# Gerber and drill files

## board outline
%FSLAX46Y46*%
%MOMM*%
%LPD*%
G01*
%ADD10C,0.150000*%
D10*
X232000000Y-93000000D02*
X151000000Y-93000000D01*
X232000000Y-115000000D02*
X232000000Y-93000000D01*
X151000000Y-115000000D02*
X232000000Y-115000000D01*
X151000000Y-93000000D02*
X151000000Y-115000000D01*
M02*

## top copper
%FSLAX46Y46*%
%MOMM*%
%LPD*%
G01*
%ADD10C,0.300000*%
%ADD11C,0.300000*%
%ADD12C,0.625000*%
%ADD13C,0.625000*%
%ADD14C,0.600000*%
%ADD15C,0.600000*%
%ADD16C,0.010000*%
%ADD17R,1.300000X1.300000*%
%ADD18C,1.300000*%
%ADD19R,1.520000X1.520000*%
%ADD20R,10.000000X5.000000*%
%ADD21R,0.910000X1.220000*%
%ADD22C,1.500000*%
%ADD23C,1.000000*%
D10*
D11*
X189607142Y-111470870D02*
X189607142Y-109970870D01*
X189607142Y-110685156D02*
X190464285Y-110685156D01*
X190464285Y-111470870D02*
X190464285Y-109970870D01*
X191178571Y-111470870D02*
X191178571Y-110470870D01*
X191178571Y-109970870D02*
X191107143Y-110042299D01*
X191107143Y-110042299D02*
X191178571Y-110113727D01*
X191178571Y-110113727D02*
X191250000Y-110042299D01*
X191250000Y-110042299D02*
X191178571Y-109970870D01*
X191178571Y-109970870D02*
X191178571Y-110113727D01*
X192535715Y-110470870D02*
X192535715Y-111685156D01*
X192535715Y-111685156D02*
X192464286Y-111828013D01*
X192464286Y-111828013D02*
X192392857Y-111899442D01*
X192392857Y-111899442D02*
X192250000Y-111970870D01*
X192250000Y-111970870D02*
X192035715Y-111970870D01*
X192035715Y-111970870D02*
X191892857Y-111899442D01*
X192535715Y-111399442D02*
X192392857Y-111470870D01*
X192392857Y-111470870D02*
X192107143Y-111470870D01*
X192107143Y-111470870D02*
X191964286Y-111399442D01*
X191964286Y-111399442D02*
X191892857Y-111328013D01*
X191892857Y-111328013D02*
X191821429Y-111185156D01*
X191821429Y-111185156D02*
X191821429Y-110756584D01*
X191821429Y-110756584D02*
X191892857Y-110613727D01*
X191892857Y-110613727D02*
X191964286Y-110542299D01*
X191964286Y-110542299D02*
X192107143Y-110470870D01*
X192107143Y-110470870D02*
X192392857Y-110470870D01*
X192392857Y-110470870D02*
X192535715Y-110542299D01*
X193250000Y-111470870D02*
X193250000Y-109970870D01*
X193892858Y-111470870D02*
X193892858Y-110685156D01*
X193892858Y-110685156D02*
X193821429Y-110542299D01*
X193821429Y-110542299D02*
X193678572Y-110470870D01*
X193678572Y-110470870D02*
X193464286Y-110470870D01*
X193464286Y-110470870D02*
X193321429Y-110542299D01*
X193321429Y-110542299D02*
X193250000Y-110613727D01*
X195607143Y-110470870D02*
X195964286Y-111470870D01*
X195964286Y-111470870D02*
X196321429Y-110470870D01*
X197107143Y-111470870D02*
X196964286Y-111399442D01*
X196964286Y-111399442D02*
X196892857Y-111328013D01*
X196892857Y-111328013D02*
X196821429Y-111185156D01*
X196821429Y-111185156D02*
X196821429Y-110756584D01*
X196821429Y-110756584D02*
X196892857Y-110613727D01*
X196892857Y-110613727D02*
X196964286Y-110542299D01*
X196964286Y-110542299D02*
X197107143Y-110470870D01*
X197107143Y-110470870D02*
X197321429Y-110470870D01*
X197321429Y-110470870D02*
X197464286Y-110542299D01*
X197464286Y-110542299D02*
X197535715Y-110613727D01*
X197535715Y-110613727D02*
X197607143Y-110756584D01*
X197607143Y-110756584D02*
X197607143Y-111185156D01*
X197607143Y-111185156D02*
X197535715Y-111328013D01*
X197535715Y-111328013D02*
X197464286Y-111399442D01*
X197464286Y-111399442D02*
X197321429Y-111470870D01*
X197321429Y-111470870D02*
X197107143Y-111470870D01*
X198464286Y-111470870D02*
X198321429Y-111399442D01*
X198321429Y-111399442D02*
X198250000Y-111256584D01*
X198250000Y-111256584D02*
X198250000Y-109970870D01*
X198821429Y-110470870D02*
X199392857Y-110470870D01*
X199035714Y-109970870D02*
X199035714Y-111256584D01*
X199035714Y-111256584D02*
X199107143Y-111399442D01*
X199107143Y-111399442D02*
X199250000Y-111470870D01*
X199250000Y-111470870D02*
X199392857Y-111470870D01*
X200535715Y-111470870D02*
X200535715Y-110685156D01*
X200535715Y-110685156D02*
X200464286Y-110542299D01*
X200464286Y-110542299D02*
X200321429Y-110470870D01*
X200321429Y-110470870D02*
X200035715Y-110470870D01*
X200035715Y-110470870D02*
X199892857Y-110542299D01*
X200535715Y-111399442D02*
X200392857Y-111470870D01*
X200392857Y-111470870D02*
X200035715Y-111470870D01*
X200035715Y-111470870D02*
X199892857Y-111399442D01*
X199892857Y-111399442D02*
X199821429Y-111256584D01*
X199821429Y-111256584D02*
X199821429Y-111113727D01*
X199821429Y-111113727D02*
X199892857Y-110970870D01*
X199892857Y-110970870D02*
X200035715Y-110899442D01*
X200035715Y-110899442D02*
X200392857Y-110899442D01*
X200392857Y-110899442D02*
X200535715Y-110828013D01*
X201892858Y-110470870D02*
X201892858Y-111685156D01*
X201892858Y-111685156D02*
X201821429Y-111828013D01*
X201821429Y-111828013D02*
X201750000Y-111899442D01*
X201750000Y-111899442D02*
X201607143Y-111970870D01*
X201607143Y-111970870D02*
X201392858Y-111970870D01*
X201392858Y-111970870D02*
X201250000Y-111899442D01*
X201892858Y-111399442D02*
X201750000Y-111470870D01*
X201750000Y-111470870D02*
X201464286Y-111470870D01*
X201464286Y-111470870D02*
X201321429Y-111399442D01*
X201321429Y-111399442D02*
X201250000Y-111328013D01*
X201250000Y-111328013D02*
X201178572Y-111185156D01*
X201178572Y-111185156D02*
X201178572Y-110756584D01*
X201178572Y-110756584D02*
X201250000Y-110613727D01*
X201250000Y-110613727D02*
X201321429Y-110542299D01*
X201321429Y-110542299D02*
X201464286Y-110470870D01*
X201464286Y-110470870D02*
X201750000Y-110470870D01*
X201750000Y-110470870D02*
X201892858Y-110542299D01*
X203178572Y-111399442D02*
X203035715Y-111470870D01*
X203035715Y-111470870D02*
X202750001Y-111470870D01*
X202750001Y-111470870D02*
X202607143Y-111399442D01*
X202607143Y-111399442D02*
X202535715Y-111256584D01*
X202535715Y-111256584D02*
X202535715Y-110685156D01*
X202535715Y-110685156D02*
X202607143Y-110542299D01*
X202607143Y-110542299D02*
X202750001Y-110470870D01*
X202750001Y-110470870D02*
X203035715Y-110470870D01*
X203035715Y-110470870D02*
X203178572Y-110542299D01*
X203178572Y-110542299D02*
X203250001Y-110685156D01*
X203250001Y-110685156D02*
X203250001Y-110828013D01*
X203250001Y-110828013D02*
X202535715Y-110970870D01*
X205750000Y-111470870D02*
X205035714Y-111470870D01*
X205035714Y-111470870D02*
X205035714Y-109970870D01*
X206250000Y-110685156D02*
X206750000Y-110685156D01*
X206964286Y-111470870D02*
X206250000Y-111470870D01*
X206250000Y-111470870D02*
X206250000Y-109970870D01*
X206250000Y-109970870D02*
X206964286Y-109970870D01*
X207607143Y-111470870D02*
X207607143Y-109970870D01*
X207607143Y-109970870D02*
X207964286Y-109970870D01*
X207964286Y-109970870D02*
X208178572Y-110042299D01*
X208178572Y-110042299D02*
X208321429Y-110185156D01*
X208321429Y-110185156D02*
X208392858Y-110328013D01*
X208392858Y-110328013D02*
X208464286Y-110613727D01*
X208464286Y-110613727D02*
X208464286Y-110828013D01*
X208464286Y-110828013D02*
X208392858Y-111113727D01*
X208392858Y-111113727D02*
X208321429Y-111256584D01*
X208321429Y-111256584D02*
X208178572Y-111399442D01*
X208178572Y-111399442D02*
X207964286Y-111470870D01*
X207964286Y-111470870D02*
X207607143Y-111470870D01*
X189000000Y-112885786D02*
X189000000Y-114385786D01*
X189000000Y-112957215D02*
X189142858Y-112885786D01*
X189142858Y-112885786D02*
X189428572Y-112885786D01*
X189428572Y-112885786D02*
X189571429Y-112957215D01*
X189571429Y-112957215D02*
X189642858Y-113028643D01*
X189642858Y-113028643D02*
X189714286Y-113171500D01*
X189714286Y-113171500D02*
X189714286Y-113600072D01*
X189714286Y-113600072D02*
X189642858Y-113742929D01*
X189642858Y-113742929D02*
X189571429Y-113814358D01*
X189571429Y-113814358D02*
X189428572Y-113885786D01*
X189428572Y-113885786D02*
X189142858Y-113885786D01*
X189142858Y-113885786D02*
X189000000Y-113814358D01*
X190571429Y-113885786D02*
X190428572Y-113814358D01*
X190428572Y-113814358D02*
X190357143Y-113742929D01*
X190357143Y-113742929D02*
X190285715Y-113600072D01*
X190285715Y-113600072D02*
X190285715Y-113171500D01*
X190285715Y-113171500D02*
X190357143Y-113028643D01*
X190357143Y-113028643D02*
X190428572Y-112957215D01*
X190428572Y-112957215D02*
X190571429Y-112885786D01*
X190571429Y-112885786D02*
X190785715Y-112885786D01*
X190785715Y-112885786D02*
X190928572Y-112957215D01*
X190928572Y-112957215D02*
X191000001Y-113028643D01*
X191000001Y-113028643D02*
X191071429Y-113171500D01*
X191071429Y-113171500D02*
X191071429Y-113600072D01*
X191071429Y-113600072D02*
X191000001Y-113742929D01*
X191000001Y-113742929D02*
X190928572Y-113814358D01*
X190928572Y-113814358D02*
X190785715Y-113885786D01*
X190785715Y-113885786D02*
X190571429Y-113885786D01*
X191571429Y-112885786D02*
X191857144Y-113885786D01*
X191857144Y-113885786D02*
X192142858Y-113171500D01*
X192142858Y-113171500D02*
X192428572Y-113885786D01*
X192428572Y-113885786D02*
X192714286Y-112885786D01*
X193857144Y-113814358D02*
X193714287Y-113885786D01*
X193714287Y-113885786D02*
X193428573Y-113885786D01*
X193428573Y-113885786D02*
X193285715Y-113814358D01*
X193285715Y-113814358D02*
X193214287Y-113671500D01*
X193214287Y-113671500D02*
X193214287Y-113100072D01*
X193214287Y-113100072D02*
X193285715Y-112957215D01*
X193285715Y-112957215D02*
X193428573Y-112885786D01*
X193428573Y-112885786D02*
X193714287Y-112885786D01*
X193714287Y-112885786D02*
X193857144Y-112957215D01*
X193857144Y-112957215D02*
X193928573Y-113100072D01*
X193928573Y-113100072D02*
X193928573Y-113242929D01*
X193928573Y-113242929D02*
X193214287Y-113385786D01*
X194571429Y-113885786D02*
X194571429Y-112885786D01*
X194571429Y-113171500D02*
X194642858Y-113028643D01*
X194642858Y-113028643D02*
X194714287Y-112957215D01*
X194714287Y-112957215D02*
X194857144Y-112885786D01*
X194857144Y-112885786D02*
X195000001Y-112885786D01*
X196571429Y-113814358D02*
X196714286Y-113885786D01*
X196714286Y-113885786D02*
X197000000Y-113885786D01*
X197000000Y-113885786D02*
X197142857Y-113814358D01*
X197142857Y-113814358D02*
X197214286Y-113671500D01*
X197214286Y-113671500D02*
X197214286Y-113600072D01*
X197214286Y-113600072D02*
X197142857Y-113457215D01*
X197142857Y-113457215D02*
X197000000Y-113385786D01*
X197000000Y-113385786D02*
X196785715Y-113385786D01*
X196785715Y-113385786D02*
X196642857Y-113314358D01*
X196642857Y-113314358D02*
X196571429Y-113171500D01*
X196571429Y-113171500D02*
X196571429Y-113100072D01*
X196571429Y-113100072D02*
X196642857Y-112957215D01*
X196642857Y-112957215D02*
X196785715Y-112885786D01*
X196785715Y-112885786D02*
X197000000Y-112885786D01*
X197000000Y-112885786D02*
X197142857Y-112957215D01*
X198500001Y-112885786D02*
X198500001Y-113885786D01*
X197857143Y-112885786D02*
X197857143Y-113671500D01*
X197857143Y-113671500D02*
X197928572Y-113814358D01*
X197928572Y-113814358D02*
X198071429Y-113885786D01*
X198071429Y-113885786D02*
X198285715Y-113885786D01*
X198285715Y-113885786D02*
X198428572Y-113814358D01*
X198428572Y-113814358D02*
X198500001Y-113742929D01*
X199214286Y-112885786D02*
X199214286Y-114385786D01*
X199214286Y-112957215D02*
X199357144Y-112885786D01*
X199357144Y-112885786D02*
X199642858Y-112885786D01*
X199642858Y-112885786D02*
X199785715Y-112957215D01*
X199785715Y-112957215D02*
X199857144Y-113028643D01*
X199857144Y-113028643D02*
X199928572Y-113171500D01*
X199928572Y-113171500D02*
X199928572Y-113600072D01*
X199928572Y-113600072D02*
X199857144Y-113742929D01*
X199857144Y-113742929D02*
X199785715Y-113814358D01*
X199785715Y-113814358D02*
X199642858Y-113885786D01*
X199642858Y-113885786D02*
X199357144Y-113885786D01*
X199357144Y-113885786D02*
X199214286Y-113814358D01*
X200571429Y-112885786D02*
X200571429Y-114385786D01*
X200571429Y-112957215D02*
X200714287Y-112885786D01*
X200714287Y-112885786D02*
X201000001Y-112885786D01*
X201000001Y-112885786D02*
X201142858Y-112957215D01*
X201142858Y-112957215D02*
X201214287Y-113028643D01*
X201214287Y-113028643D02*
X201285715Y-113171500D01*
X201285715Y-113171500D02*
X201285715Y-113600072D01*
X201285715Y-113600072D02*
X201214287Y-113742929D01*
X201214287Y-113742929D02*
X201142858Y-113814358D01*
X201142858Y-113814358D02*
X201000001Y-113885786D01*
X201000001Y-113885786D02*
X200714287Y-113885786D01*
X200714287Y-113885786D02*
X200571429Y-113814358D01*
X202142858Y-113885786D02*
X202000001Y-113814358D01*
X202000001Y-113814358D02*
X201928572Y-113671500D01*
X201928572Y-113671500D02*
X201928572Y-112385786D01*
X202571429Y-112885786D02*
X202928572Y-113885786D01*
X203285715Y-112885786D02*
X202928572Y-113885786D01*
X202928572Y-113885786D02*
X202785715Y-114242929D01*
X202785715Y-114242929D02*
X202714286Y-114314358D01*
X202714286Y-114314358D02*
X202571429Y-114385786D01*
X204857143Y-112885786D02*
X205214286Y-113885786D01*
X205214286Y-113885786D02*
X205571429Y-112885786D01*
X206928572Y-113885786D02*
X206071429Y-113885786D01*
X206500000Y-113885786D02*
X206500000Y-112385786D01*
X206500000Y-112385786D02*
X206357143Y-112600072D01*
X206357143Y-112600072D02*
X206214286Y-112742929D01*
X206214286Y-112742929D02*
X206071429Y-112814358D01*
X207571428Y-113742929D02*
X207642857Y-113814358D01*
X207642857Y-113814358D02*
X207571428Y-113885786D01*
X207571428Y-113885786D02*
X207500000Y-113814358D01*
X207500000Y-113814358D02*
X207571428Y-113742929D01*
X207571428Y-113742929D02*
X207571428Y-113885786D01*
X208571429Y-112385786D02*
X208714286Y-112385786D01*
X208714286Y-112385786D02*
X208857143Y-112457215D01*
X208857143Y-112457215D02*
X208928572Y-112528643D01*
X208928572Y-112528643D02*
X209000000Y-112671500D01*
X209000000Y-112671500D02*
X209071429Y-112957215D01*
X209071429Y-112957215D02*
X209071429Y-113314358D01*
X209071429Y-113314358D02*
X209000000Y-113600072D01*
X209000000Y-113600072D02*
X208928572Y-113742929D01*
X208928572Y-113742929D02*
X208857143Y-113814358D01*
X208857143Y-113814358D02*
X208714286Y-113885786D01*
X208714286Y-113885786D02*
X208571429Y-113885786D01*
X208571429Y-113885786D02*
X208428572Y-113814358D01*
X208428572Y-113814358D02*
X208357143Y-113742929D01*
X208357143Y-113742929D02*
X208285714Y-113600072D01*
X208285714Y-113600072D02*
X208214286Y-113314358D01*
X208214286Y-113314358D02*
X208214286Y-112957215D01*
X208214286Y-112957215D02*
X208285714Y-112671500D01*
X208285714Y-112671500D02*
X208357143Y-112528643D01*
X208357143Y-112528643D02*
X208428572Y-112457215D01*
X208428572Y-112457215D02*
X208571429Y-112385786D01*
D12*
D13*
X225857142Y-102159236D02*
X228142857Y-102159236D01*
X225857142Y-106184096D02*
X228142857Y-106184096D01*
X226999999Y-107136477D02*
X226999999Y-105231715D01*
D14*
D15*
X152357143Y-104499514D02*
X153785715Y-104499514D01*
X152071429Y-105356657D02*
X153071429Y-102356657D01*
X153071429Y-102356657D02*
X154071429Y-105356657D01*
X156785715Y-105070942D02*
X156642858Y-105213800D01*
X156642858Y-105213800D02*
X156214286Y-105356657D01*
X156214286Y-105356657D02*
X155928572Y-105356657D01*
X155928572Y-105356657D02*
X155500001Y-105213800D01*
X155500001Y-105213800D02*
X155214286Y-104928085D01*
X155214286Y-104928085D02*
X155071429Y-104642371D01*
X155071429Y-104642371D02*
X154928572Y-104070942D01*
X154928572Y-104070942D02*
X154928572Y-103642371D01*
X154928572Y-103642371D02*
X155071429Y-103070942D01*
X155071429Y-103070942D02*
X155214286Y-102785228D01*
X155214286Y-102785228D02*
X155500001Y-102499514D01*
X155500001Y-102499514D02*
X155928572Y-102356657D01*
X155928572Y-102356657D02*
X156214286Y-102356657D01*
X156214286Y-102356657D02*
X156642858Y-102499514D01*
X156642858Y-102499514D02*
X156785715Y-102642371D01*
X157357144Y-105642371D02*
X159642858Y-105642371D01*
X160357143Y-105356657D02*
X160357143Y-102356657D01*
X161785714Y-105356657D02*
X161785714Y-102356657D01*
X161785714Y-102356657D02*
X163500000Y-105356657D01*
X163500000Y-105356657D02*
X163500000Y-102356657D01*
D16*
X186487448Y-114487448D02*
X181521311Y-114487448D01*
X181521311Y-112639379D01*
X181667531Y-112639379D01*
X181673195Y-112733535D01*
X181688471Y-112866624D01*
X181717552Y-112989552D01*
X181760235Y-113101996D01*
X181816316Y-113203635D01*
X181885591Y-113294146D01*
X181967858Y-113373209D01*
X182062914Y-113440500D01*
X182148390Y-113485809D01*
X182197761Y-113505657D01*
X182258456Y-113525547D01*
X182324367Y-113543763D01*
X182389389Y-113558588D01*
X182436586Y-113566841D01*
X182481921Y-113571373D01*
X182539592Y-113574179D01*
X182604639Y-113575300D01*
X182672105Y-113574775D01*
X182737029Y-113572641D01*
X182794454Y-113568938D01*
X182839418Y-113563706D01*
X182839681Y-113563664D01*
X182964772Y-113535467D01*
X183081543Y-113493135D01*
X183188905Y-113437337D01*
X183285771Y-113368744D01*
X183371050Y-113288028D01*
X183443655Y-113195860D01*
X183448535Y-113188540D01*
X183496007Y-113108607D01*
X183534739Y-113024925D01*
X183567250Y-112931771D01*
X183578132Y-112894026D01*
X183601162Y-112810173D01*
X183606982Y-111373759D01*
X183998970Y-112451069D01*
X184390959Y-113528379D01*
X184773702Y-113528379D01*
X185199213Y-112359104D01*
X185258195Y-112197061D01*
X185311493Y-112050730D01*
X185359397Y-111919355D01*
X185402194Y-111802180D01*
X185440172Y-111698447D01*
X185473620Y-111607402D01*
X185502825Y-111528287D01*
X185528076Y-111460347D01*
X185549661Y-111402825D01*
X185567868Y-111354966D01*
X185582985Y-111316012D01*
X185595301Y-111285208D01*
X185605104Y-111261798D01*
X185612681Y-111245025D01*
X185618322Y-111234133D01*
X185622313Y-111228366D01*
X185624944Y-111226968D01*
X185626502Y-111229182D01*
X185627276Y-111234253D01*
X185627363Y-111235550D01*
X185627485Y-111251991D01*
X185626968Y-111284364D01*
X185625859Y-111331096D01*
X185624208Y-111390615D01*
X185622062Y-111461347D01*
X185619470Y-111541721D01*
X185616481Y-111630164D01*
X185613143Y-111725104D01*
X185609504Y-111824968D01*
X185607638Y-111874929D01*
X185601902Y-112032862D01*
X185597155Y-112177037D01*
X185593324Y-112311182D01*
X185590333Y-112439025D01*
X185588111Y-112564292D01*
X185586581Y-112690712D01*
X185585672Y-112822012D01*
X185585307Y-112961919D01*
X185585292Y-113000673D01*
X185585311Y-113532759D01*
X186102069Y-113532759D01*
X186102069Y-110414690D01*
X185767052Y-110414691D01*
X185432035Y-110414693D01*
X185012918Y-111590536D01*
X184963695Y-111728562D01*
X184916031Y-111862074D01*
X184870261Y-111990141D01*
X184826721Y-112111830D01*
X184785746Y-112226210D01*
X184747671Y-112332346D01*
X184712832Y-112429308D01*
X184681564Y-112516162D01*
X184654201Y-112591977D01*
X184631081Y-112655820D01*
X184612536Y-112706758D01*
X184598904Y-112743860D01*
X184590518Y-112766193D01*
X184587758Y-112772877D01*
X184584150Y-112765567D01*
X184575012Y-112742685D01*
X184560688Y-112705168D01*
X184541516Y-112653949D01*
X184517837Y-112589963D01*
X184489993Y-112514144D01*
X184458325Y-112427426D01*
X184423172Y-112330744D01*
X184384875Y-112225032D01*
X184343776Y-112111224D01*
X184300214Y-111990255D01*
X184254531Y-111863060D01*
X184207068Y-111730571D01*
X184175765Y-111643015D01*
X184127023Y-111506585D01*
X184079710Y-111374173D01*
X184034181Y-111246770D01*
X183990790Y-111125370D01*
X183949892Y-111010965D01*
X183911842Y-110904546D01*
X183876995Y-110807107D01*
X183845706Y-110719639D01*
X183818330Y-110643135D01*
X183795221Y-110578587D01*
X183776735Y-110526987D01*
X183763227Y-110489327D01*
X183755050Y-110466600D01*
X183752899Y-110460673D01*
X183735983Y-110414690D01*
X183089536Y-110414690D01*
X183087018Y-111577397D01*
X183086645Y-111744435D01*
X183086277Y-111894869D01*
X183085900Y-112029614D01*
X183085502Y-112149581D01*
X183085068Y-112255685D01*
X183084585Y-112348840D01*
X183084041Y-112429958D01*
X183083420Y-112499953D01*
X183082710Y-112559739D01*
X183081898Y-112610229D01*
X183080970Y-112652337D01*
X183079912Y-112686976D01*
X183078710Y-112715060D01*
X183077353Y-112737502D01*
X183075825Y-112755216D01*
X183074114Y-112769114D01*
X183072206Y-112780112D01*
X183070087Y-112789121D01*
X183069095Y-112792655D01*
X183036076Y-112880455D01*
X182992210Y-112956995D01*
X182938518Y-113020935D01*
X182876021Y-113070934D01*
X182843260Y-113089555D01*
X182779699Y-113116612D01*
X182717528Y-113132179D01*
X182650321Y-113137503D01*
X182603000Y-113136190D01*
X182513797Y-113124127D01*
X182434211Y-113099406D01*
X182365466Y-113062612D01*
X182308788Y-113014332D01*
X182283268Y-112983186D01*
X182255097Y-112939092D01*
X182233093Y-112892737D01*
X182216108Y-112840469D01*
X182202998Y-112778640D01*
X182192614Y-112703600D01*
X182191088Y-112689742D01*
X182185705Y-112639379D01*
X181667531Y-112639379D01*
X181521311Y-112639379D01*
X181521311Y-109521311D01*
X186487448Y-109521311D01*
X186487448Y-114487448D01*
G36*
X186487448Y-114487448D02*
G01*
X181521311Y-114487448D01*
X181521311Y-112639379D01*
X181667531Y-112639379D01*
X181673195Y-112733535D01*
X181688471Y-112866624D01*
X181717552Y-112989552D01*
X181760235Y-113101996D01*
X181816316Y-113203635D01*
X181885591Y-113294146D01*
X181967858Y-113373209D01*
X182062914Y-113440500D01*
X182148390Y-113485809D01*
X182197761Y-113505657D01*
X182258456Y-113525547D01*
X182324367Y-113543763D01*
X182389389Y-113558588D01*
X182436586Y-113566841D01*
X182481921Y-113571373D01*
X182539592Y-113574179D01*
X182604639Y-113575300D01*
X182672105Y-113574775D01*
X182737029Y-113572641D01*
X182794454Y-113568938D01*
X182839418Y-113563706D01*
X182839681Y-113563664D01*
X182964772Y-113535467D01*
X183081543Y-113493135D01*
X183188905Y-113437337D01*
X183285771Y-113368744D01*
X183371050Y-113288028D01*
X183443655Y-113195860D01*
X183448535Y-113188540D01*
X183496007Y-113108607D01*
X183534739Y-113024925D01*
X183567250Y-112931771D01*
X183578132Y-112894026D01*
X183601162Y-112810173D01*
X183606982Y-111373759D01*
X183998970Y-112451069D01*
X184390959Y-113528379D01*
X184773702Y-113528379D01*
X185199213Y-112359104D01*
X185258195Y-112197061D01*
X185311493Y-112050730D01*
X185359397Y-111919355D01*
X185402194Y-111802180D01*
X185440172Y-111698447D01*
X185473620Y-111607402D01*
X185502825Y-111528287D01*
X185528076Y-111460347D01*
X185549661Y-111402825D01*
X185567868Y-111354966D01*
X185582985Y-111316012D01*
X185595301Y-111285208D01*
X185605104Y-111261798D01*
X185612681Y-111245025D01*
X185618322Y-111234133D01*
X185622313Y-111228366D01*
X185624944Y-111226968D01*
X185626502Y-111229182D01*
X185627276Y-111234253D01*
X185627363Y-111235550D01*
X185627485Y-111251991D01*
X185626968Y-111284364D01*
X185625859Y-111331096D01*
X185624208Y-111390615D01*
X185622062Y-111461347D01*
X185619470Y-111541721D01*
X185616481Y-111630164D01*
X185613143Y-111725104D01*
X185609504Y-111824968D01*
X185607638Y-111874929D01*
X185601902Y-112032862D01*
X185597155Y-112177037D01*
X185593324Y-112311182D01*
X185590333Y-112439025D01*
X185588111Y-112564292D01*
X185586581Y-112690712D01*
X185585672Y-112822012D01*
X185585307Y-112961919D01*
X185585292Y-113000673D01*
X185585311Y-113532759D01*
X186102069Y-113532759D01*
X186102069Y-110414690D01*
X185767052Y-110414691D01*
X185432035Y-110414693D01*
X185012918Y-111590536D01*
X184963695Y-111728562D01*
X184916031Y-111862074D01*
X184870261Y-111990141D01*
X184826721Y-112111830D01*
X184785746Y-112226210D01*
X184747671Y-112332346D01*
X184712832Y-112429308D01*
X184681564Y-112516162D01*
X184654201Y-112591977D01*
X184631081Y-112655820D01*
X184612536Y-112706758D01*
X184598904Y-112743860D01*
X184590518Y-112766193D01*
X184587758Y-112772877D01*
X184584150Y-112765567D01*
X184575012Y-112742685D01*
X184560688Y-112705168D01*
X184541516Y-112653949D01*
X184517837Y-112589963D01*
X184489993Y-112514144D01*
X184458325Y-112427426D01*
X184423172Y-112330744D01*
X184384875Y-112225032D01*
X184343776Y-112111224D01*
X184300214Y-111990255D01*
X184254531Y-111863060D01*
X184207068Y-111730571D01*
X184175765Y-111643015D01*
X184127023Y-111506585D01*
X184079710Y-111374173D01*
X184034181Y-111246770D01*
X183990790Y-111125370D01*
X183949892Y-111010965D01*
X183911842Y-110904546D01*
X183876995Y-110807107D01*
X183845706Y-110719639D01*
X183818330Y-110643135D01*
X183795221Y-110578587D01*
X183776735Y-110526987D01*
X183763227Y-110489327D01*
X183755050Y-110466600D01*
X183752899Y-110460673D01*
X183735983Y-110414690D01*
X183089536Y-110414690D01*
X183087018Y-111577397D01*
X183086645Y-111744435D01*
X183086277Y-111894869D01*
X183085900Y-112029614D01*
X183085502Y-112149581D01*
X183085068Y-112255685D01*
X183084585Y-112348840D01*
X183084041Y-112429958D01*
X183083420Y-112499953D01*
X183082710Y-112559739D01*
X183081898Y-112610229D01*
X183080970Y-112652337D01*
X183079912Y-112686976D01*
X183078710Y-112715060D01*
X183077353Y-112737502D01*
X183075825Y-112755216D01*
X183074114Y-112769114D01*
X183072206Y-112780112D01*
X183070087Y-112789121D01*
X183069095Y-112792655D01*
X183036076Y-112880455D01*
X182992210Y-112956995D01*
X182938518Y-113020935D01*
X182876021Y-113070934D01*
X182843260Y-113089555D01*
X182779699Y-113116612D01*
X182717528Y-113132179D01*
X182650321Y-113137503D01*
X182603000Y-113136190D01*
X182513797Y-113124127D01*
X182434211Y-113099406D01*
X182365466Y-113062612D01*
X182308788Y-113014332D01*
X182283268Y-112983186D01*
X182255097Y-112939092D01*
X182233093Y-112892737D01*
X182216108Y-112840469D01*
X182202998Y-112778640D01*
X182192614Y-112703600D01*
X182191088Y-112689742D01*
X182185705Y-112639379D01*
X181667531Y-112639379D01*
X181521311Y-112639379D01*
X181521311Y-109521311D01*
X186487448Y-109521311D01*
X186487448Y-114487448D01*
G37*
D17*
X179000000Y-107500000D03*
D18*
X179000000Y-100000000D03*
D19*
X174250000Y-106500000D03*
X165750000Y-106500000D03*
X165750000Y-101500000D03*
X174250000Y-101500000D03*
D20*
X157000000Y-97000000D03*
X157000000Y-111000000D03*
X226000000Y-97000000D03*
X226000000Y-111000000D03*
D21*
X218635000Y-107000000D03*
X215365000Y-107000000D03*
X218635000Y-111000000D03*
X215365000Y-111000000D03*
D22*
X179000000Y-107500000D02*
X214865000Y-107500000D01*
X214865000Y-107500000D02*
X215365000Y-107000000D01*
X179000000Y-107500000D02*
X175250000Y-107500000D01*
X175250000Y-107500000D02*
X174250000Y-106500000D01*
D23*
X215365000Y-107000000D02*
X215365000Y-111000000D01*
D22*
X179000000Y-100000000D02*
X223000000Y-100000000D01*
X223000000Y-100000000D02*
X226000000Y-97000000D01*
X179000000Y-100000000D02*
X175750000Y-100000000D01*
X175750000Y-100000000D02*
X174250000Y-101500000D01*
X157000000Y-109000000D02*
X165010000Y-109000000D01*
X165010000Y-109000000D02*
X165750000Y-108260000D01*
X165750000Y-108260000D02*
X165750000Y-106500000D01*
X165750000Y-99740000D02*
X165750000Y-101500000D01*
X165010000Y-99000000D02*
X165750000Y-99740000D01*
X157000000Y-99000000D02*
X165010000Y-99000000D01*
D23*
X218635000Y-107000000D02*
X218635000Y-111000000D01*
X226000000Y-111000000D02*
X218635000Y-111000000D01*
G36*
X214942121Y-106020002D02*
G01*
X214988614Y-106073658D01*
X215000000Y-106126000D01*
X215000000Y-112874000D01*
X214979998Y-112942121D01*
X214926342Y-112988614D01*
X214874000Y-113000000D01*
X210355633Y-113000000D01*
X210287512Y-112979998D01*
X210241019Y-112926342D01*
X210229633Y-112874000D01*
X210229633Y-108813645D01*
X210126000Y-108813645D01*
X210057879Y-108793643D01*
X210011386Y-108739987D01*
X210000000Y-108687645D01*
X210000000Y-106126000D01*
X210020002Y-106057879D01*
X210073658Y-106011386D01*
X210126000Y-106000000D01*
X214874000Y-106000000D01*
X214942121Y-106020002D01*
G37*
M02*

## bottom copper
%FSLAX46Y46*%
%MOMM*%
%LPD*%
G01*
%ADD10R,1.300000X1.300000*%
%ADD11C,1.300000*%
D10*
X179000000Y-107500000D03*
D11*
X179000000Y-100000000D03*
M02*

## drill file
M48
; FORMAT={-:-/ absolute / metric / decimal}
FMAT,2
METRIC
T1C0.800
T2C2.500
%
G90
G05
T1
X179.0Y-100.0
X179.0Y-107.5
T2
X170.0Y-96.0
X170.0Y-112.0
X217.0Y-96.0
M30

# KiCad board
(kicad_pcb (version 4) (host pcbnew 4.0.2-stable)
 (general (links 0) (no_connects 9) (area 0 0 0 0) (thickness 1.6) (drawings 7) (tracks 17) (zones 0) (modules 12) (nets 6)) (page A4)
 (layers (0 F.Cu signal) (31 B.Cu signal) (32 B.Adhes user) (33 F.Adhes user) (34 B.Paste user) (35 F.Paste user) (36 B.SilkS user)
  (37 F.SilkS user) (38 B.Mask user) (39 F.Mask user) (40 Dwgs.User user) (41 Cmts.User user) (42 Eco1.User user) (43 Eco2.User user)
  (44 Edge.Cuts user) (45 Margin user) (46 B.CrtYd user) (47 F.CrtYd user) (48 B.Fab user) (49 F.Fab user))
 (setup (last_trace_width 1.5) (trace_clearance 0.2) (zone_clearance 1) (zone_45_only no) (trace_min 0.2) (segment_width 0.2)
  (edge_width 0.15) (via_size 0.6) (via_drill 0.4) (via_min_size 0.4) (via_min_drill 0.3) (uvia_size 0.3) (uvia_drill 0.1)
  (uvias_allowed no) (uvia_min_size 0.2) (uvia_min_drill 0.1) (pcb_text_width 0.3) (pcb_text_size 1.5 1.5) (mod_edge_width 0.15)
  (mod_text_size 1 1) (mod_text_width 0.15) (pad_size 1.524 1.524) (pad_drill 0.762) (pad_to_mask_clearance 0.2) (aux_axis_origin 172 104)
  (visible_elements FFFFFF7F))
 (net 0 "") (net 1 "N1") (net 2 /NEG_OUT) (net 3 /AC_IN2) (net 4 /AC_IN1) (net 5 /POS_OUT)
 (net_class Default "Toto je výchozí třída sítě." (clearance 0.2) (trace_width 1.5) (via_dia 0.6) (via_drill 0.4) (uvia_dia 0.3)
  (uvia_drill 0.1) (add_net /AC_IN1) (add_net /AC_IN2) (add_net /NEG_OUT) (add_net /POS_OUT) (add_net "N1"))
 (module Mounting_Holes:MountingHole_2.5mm (layer F.Cu) (at 217 96)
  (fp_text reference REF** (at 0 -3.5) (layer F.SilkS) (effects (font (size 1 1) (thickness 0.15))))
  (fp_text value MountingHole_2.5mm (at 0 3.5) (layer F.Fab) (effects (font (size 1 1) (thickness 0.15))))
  (pad 1 np_thru_hole circle (at 0 0) (size 2.5 2.5) (drill 2.5) (layers *.Cu *.Mask F.SilkS)))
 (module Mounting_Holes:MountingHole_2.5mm (layer F.Cu) (at 170 96)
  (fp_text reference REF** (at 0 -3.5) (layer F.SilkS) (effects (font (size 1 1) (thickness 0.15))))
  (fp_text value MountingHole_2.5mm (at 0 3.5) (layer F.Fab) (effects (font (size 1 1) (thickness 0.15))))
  (pad 1 np_thru_hole circle (at 0 0) (size 2.5 2.5) (drill 2.5) (layers *.Cu *.Mask F.SilkS)))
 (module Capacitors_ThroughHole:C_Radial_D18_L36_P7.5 (layer F.Cu) (at 179 107.5 90)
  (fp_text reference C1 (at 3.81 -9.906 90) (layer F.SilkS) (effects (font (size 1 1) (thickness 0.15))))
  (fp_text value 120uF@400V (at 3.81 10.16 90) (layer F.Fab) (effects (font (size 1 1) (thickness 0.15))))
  (pad 1 thru_hole rect (at 0 0 90) (size 1.3 1.3) (drill 0.8) (layers *.Cu *.Mask F.SilkS) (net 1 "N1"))
  (pad 2 thru_hole circle (at 7.5 0 90) (size 1.3 1.3) (drill 0.8) (layers *.Cu *.Mask F.SilkS) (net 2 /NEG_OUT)))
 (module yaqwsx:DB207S (layer F.Cu) (at 170 104 270)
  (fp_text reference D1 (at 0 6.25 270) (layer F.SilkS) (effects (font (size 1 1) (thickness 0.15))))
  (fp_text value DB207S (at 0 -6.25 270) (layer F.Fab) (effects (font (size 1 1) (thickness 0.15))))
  (pad 3 smd rect (at 2.5 -4.25 270) (size 1.52 1.52) (layers F.Cu F.Paste F.Mask) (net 1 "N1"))
  (pad 4 smd rect (at 2.5 4.25 270) (size 1.52 1.52) (layers F.Cu F.Paste F.Mask) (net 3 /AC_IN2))
  (pad 2 smd rect (at -2.5 4.25 270) (size 1.52 1.52) (layers F.Cu F.Paste F.Mask) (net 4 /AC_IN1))
  (pad 1 smd rect (at -2.5 -4.25 270) (size 1.52 1.52) (layers F.Cu F.Paste F.Mask) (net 2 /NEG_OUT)))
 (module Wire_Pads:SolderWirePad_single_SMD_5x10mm (layer F.Cu) (at 157 97 90)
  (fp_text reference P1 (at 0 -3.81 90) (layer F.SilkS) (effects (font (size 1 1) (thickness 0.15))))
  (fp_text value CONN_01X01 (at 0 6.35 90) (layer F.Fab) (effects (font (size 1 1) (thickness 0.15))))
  (pad 1 smd rect (at 0 0 90) (size 5 10) (layers F.Cu F.Paste F.Mask) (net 4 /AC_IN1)))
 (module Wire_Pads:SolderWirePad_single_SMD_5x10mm (layer F.Cu) (at 157 111 90)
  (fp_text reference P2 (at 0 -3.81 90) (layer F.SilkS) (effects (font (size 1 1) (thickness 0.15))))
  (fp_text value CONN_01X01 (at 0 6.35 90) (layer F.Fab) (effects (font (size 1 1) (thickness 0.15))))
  (pad 1 smd rect (at 0 0 90) (size 5 10) (layers F.Cu F.Paste F.Mask) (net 3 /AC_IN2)))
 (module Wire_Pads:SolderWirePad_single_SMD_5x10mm (layer F.Cu) (at 226 97 90)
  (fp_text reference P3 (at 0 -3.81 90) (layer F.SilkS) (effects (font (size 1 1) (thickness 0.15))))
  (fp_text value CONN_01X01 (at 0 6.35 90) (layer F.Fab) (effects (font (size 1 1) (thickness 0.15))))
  (pad 1 smd rect (at 0 0 90) (size 5 10) (layers F.Cu F.Paste F.Mask) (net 2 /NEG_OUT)))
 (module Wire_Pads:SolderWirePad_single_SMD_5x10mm (layer F.Cu) (at 226 111 90)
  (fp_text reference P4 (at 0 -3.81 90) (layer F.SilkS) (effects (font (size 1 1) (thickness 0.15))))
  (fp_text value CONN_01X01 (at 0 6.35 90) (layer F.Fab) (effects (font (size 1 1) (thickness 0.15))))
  (pad 1 smd rect (at 0 0 90) (size 5 10) (layers F.Cu F.Paste F.Mask) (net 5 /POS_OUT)))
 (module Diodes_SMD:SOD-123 (layer F.Cu) (at 217 107 180)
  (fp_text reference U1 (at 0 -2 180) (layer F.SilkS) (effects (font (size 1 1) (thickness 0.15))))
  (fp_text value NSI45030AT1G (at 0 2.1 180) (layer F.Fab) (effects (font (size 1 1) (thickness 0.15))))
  (pad 1 smd rect (at -1.635 0 180) (size 0.91 1.22) (layers F.Cu F.Paste F.Mask) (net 5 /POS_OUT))
  (pad 2 smd rect (at 1.635 0 180) (size 0.91 1.22) (layers F.Cu F.Paste F.Mask) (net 1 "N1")))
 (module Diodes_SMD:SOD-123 (layer F.Cu) (at 217 111 180)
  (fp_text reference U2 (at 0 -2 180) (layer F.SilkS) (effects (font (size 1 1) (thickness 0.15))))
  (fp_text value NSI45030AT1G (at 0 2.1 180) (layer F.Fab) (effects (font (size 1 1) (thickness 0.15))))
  (pad 1 smd rect (at -1.635 0 180) (size 0.91 1.22) (layers F.Cu F.Paste F.Mask) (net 5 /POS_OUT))
  (pad 2 smd rect (at 1.635 0 180) (size 0.91 1.22) (layers F.Cu F.Paste F.Mask) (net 1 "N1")))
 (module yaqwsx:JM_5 (layer F.Cu) (at 184 112)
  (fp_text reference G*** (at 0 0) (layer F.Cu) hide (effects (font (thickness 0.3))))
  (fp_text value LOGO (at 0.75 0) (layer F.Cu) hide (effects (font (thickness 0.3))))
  (fp_poly
   (pts (xy 2.487448 2.487448) (xy -2.478689 2.487448) (xy -2.478689 0.639379) (xy -2.332469 0.639379) (xy -2.326805 0.733535)
    (xy -2.311529 0.866624) (xy -2.282448 0.989552) (xy -2.239765 1.101996) (xy -2.183684 1.203635) (xy -2.114409 1.294146)
    (xy -2.032142 1.373209) (xy -1.937086 1.4405) (xy -1.85161 1.485809) (xy -1.802239 1.505657) (xy -1.741544 1.525547)
    (xy -1.675633 1.543763) (xy -1.610611 1.558588) (xy -1.563414 1.566841) (xy -1.518079 1.571373) (xy -1.460408 1.574179)
    (xy -1.395361 1.5753) (xy -1.327895 1.574775) (xy -1.262971 1.572641) (xy -1.205546 1.568938) (xy -1.160582 1.563706)
    (xy -1.160319 1.563664) (xy -1.035228 1.535467) (xy -0.918457 1.493135) (xy -0.811095 1.437337) (xy -0.714229 1.368744)
    (xy -0.62895 1.288028) (xy -0.556345 1.19586) (xy -0.551465 1.18854) (xy -0.503993 1.108607) (xy -0.465261 1.024925)
    (xy -0.43275 0.931771) (xy -0.421868 0.894026) (xy -0.398838 0.810173) (xy -0.393018 -0.626241) (xy -0.00103 0.451069)
    (xy 0.390959 1.528379) (xy 0.773702 1.528379) (xy 1.199213 0.359104) (xy 1.258195 0.197061) (xy 1.311493 0.05073)
    (xy 1.359397 -0.080645) (xy 1.402194 -0.19782) (xy 1.440172 -0.301553) (xy 1.47362 -0.392598) (xy 1.502825 -0.471713)
    (xy 1.528076 -0.539653) (xy 1.549661 -0.597175) (xy 1.567868 -0.645034) (xy 1.582985 -0.683988) (xy 1.595301 -0.714792)
    (xy 1.605104 -0.738202) (xy 1.612681 -0.754975) (xy 1.618322 -0.765867) (xy 1.622313 -0.771634) (xy 1.624944 -0.773032)
    (xy 1.626502 -0.770818) (xy 1.627276 -0.765747) (xy 1.627363 -0.76445) (xy 1.627485 -0.748009) (xy 1.626968 -0.715636)
    (xy 1.625859 -0.668904) (xy 1.624208 -0.609385) (xy 1.622062 -0.538653) (xy 1.61947 -0.458279) (xy 1.616481 -0.369836)
    (xy 1.613143 -0.274896) (xy 1.609504 -0.175032) (xy 1.607638 -0.125071) (xy 1.601902 0.032862) (xy 1.597155 0.177037)
    (xy 1.593324 0.311182) (xy 1.590333 0.439025) (xy 1.588111 0.564292) (xy 1.586581 0.690712) (xy 1.585672 0.822012)
    (xy 1.585307 0.961919) (xy 1.585292 1.000673) (xy 1.585311 1.532759) (xy 2.102069 1.532759) (xy 2.102069 -1.58531)
    (xy 1.767052 -1.585309) (xy 1.432035 -1.585307) (xy 1.012918 -0.409464) (xy 0.963695 -0.271438) (xy 0.916031 -0.137926)
    (xy 0.870261 -0.009859) (xy 0.826721 0.11183) (xy 0.785746 0.22621) (xy 0.747671 0.332346) (xy 0.712832 0.429308) (xy 0.681564 0.516162)
    (xy 0.654201 0.591977) (xy 0.631081 0.65582) (xy 0.612536 0.706758) (xy 0.598904 0.74386) (xy 0.590518 0.766193) (xy 0.587758 0.772877)
    (xy 0.58415 0.765567) (xy 0.575012 0.742685) (xy 0.560688 0.705168) (xy 0.541516 0.653949) (xy 0.517837 0.589963) (xy 0.489993 0.514144)
    (xy 0.458325 0.427426) (xy 0.423172 0.330744) (xy 0.384875 0.225032) (xy 0.343776 0.111224) (xy 0.300214 -0.009745)
    (xy 0.254531 -0.13694) (xy 0.207068 -0.269429) (xy 0.175765 -0.356985) (xy 0.127023 -0.493415) (xy 0.07971 -0.625827)
    (xy 0.034181 -0.75323) (xy -0.00921 -0.87463) (xy -0.050108 -0.989035) (xy -0.088158 -1.095454) (xy -0.123005 -1.192893)
    (xy -0.154294 -1.280361) (xy -0.18167 -1.356865) (xy -0.204779 -1.421413) (xy -0.223265 -1.473013) (xy -0.236773 -1.510673)
    (xy -0.24495 -1.5334) (xy -0.247101 -1.539327) (xy -0.264017 -1.58531) (xy -0.910464 -1.58531) (xy -0.912982 -0.422603)
    (xy -0.913355 -0.255565) (xy -0.913723 -0.105131) (xy -0.9141 0.029614) (xy -0.914498 0.149581) (xy -0.914932 0.255685)
    (xy -0.915415 0.34884) (xy -0.915959 0.429958) (xy -0.91658 0.499953) (xy -0.91729 0.559739) (xy -0.918102 0.610229)
    (xy -0.91903 0.652337) (xy -0.920088 0.686976) (xy -0.92129 0.71506) (xy -0.922647 0.737502) (xy -0.924175 0.755216)
    (xy -0.925886 0.769114) (xy -0.927794 0.780112) (xy -0.929913 0.789121) (xy -0.930905 0.792655) (xy -0.963924 0.880455)
    (xy -1.00779 0.956995) (xy -1.061482 1.020935) (xy -1.123979 1.070934) (xy -1.15674 1.089555) (xy -1.220301 1.116612)
    (xy -1.282472 1.132179) (xy -1.349679 1.137503) (xy -1.397 1.13619) (xy -1.486203 1.124127) (xy -1.565789 1.099406)
    (xy -1.634534 1.062612) (xy -1.691212 1.014332) (xy -1.716732 0.983186) (xy -1.744903 0.939092) (xy -1.766907 0.892737)
    (xy -1.783892 0.840469) (xy -1.797002 0.77864) (xy -1.807386 0.7036) (xy -1.808912 0.689742) (xy -1.814295 0.639379)
    (xy -2.332469 0.639379) (xy -2.478689 0.639379) (xy -2.478689 -2.478689) (xy 2.487448 -2.478689) (xy 2.487448 2.487448))
   (layer F.Cu) (width 0.01)))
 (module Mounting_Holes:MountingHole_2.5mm (layer F.Cu) (at 170 112)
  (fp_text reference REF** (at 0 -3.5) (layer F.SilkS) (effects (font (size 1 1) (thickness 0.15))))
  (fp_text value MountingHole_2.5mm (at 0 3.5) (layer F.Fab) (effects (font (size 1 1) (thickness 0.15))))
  (pad 1 np_thru_hole circle (at 0 0) (size 2.5 2.5) (drill 2.5) (layers *.Cu *.Mask F.SilkS)))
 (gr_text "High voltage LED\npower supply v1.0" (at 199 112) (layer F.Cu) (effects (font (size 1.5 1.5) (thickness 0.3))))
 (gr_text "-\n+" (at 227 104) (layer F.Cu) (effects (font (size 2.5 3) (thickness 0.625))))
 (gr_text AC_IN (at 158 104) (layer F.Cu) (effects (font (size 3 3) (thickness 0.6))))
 (gr_line (start 232 93) (end 151 93) (layer Edge.Cuts) (width 0.15))
 (gr_line (start 232 115) (end 232 93) (layer Edge.Cuts) (width 0.15))
 (gr_line (start 151 115) (end 232 115) (layer Edge.Cuts) (width 0.15))
 (gr_line (start 151 93) (end 151 115) (layer Edge.Cuts) (width 0.15))
 (segment (start 179 107.5) (end 214.865 107.5) (width 1.5) (layer F.Cu) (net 1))
 (segment (start 214.865 107.5) (end 215.365 107) (width 1.5) (layer F.Cu) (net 1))
 (segment (start 179 107.5) (end 175.25 107.5) (width 1.5) (layer F.Cu) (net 1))
 (segment (start 175.25 107.5) (end 174.25 106.5) (width 1.5) (layer F.Cu) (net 1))
 (segment (start 215.365 107) (end 215.365 111) (width 1) (layer F.Cu) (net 1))
 (segment (start 179 100) (end 223 100) (width 1.5) (layer F.Cu) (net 2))
 (segment (start 223 100) (end 226 97) (width 1.5) (layer F.Cu) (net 2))
 (segment (start 179 100) (end 175.75 100) (width 1.5) (layer F.Cu) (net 2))
 (segment (start 175.75 100) (end 174.25 101.5) (width 1.5) (layer F.Cu) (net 2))
 (segment (start 157 109) (end 165.01 109) (width 1.5) (layer F.Cu) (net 3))
 (segment (start 165.01 109) (end 165.75 108.26) (width 1.5) (layer F.Cu) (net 3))
 (segment (start 165.75 108.26) (end 165.75 106.5) (width 1.5) (layer F.Cu) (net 3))
 (segment (start 165.75 99.74) (end 165.75 101.5) (width 1.5) (layer F.Cu) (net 4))
 (segment (start 165.01 99) (end 165.75 99.74) (width 1.5) (layer F.Cu) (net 4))
 (segment (start 157 99) (end 165.01 99) (width 1.5) (layer F.Cu) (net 4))
 (segment (start 218.635 107) (end 218.635 111) (width 1) (layer F.Cu) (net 5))
 (segment (start 226 111) (end 218.635 111) (width 1) (layer F.Cu) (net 5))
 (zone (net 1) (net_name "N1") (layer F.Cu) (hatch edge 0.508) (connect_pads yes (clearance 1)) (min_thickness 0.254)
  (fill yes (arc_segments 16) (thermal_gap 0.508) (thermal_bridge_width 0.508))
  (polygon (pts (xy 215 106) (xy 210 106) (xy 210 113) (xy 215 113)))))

